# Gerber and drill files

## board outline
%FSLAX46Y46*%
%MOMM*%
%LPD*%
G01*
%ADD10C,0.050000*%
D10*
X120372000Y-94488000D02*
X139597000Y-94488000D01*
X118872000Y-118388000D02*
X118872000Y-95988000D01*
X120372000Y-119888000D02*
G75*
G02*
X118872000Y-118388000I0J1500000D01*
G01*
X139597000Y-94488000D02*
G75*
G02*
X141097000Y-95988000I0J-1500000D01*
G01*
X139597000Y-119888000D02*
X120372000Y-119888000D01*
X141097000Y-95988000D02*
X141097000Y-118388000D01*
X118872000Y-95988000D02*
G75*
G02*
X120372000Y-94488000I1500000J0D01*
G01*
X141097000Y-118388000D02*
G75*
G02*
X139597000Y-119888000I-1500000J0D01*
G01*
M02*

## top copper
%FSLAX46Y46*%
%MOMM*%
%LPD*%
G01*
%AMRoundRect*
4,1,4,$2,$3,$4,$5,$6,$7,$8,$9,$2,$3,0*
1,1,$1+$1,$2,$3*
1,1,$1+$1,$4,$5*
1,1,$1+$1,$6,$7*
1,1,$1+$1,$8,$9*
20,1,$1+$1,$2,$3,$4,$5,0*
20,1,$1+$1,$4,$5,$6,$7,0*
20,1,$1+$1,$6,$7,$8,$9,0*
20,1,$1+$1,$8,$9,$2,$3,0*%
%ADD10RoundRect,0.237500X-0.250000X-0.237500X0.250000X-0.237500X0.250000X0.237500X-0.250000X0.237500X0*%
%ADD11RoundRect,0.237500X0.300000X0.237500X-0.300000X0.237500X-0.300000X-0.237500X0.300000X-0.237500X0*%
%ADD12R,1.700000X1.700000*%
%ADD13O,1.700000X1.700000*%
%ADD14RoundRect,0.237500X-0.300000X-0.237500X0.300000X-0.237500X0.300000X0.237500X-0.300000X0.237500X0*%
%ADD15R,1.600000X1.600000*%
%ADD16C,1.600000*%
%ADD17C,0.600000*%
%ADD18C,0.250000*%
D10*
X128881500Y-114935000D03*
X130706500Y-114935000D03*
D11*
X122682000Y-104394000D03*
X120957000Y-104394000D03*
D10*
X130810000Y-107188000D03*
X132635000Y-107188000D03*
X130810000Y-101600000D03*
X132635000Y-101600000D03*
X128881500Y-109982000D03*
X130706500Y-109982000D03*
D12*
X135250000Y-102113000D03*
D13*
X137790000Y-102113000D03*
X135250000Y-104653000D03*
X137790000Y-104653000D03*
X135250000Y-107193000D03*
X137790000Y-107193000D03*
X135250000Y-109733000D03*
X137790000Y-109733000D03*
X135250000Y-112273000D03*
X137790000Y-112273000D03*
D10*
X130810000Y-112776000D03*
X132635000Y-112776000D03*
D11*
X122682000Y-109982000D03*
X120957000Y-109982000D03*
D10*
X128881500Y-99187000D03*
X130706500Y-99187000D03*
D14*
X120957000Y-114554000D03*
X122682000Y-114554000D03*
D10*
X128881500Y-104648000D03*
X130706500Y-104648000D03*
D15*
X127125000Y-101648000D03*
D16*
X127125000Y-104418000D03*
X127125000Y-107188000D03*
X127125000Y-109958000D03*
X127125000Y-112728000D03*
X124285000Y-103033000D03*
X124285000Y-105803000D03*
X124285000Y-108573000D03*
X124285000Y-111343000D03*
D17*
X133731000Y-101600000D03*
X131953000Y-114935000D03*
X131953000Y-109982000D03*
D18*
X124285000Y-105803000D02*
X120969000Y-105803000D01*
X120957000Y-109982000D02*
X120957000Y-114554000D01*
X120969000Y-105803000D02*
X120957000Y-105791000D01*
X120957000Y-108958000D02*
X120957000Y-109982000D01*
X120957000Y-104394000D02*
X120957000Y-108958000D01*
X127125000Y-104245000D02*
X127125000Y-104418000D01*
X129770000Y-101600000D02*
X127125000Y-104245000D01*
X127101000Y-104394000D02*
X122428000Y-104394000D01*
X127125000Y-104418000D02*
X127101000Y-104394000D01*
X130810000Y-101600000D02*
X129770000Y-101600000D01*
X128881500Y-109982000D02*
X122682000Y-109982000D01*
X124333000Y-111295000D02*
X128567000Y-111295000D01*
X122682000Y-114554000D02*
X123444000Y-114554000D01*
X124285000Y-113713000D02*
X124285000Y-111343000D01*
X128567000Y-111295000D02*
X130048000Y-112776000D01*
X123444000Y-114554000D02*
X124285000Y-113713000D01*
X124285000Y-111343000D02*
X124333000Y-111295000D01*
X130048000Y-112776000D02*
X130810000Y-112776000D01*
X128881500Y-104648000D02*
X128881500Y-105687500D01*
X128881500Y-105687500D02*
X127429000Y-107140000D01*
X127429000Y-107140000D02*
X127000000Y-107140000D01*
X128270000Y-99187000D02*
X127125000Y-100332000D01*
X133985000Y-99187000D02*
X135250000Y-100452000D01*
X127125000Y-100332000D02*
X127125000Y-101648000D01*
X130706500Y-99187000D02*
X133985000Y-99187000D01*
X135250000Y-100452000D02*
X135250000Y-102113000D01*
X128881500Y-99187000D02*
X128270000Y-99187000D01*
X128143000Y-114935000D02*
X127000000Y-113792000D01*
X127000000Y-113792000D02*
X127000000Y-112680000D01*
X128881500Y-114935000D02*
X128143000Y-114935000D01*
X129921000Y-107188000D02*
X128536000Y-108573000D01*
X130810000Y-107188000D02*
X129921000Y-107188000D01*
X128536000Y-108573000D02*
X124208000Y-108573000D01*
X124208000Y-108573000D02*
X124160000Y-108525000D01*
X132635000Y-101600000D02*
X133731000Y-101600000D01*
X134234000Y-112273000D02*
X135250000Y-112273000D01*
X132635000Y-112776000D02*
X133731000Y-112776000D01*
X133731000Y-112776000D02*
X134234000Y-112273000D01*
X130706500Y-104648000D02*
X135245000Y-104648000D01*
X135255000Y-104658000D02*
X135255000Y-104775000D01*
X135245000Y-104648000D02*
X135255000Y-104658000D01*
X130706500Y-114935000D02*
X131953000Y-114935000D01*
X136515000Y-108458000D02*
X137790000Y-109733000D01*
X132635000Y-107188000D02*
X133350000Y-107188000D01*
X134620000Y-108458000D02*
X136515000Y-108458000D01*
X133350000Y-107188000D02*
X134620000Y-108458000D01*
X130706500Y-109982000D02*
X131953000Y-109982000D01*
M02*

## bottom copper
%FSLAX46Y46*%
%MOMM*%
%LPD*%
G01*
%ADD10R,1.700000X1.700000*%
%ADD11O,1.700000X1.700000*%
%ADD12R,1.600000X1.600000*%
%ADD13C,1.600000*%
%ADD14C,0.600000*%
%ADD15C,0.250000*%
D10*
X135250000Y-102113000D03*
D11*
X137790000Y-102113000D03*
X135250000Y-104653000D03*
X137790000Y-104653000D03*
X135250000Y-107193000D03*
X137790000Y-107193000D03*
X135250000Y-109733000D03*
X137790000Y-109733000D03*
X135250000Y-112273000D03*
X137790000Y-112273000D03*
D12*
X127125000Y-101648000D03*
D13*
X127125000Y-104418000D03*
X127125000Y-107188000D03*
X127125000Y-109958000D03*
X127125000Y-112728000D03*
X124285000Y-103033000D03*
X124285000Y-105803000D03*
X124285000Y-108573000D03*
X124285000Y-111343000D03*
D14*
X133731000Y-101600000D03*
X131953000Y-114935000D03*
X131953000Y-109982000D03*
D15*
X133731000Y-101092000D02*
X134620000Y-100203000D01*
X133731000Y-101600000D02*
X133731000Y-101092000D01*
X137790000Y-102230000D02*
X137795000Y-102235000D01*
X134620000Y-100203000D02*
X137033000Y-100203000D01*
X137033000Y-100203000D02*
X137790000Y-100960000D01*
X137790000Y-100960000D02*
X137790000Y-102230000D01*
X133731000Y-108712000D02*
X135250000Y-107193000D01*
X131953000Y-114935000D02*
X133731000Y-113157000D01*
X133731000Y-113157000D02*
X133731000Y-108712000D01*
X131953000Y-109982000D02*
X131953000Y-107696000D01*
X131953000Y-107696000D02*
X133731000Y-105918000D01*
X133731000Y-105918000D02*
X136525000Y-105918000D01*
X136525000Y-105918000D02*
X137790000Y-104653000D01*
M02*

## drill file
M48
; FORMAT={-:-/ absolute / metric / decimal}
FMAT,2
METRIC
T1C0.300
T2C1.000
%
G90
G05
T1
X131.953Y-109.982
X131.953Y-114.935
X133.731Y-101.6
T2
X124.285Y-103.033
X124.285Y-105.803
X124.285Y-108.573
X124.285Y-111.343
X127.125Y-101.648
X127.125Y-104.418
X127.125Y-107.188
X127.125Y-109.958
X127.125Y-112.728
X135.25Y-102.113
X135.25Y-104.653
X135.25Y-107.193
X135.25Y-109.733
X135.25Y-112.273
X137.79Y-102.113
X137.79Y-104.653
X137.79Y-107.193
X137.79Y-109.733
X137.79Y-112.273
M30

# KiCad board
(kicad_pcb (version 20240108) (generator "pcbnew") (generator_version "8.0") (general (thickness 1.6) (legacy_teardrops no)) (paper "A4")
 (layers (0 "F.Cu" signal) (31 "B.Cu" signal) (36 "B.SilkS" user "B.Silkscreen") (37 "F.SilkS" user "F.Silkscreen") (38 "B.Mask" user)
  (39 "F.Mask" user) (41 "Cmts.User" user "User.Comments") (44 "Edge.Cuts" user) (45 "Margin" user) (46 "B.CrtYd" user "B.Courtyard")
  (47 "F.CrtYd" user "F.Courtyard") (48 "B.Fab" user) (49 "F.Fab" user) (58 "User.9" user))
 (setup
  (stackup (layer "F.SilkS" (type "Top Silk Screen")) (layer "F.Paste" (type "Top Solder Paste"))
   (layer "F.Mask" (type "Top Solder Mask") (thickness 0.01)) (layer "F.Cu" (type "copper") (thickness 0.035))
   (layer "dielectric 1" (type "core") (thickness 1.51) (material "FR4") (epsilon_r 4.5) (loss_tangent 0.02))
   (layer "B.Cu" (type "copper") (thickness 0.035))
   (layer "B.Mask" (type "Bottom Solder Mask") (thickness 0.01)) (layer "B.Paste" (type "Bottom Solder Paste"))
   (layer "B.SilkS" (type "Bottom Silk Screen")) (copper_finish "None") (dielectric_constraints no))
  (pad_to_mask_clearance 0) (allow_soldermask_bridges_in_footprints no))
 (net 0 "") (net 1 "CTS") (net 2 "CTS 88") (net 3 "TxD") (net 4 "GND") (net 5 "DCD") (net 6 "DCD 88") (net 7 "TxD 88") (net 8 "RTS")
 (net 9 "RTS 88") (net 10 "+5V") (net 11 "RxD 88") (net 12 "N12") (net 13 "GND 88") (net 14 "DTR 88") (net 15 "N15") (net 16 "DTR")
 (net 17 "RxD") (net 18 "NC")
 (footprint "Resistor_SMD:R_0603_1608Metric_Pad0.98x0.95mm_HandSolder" (layer "F.Cu") (at 129.794 114.935)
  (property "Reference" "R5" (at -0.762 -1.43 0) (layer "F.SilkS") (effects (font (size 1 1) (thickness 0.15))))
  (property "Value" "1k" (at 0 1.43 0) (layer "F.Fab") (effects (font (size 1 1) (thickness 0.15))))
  (pad "1" smd roundrect (at -0.9125 0) (size 0.975 0.95) (layers "F.Cu" "F.Paste" "F.Mask") (roundrect_rratio 0.25) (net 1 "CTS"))
  (pad "2" smd roundrect (at 0.9125 0) (size 0.975 0.95) (layers "F.Cu" "F.Paste" "F.Mask") (roundrect_rratio 0.25) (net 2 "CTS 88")))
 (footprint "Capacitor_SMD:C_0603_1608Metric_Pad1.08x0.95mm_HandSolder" (layer "F.Cu") (at 121.8195 104.394 180)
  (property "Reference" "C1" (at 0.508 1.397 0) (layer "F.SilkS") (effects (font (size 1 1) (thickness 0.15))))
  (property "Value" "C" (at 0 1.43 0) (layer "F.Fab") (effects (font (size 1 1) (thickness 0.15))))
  (pad "1" smd roundrect (at -0.8625 0 180) (size 1.075 0.95) (layers "F.Cu" "F.Paste" "F.Mask") (roundrect_rratio 0.25) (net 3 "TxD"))
  (pad "2" smd roundrect (at 0.8625 0 180) (size 1.075 0.95) (layers "F.Cu" "F.Paste" "F.Mask") (roundrect_rratio 0.25) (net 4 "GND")))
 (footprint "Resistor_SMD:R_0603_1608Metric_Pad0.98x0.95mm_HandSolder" (layer "F.Cu") (at 131.7225 107.188)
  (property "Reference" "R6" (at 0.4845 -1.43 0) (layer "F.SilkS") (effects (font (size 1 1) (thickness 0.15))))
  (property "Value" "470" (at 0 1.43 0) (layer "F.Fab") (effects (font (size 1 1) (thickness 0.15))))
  (pad "1" smd roundrect (at -0.9125 0) (size 0.975 0.95) (layers "F.Cu" "F.Paste" "F.Mask") (roundrect_rratio 0.25) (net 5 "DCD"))
  (pad "2" smd roundrect (at 0.9125 0) (size 0.975 0.95) (layers "F.Cu" "F.Paste" "F.Mask") (roundrect_rratio 0.25) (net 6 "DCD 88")))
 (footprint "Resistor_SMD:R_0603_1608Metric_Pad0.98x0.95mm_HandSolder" (layer "F.Cu") (at 131.7225 101.6)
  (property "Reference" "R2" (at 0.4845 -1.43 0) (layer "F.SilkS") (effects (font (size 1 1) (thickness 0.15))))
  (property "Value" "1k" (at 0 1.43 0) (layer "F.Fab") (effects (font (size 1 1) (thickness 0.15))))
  (pad "1" smd roundrect (at -0.9125 0) (size 0.975 0.95) (layers "F.Cu" "F.Paste" "F.Mask") (roundrect_rratio 0.25) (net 3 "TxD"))
  (pad "2" smd roundrect (at 0.9125 0) (size 0.975 0.95) (layers "F.Cu" "F.Paste" "F.Mask") (roundrect_rratio 0.25) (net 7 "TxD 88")))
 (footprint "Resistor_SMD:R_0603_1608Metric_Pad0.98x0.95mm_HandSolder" (layer "F.Cu") (at 129.794 109.982)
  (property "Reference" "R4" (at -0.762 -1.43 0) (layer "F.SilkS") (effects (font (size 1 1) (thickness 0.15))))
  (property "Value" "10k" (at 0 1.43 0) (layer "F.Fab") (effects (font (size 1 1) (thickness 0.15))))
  (pad "1" smd roundrect (at -0.9125 0) (size 0.975 0.95) (layers "F.Cu" "F.Paste" "F.Mask") (roundrect_rratio 0.25) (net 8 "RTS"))
  (pad "2" smd roundrect (at 0.9125 0) (size 0.975 0.95) (layers "F.Cu" "F.Paste" "F.Mask") (roundrect_rratio 0.25) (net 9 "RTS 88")))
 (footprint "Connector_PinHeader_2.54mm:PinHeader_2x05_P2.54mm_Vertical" (layer "F.Cu") (at 135.25 102.113)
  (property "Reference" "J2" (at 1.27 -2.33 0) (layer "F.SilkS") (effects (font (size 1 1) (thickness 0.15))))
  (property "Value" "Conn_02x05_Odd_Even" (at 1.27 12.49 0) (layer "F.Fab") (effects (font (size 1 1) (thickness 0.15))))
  (pad "1" thru_hole rect (at 0 0) (size 1.7 1.7) (drill 1) (layers "*.Cu" "*.Mask") (remove_unused_layers no) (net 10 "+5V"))
  (pad "2" thru_hole oval (at 2.54 0) (size 1.7 1.7) (drill 1) (layers "*.Cu" "*.Mask") (remove_unused_layers no) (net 7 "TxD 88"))
  (pad "3" thru_hole oval (at 0 2.54) (size 1.7 1.7) (drill 1) (layers "*.Cu" "*.Mask") (remove_unused_layers no) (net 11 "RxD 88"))
  (pad "4" thru_hole oval (at 2.54 2.54) (size 1.7 1.7) (drill 1) (layers "*.Cu" "*.Mask") (remove_unused_layers no) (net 9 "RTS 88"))
  (pad "5" thru_hole oval (at 0 5.08) (size 1.7 1.7) (drill 1) (layers "*.Cu" "*.Mask") (remove_unused_layers no) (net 2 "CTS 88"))
  (pad "6" thru_hole oval (at 2.54 5.08) (size 1.7 1.7) (drill 1) (layers "*.Cu" "*.Mask") (remove_unused_layers no) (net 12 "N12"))
  (pad "7" thru_hole oval (at 0 7.62) (size 1.7 1.7) (drill 1) (layers "*.Cu" "*.Mask") (remove_unused_layers no) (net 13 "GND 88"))
  (pad "8" thru_hole oval (at 2.54 7.62) (size 1.7 1.7) (drill 1) (layers "*.Cu" "*.Mask") (remove_unused_layers no) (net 6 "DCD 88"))
  (pad "9" thru_hole oval (at 0 10.16) (size 1.7 1.7) (drill 1) (layers "*.Cu" "*.Mask") (remove_unused_layers no) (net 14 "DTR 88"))
  (pad "10" thru_hole oval (at 2.54 10.16) (size 1.7 1.7) (drill 1) (layers "*.Cu" "*.Mask") (remove_unused_layers no) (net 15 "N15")))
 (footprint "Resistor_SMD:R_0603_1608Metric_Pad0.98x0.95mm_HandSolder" (layer "F.Cu") (at 131.7225 112.776)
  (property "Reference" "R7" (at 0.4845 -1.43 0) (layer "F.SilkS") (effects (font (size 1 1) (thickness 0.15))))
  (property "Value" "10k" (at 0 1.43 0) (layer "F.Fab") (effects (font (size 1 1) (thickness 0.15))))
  (pad "1" smd roundrect (at -0.9125 0) (size 0.975 0.95) (layers "F.Cu" "F.Paste" "F.Mask") (roundrect_rratio 0.25) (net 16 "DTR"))
  (pad "2" smd roundrect (at 0.9125 0) (size 0.975 0.95) (layers "F.Cu" "F.Paste" "F.Mask") (roundrect_rratio 0.25) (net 14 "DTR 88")))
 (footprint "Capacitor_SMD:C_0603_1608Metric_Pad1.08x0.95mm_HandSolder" (layer "F.Cu") (at 121.8195 109.982 180)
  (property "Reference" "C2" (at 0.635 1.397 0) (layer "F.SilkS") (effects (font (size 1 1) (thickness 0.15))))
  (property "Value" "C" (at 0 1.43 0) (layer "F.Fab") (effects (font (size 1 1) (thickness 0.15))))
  (pad "1" smd roundrect (at -0.8625 0 180) (size 1.075 0.95) (layers "F.Cu" "F.Paste" "F.Mask") (roundrect_rratio 0.25) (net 8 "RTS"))
  (pad "2" smd roundrect (at 0.8625 0 180) (size 1.075 0.95) (layers "F.Cu" "F.Paste" "F.Mask") (roundrect_rratio 0.25) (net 4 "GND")))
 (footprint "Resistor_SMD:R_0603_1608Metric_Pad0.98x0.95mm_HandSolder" (layer "F.Cu") (at 129.794 99.187)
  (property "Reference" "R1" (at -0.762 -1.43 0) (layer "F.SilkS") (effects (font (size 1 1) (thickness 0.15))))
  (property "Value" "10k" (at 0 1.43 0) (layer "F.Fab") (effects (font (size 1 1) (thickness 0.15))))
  (pad "1" smd roundrect (at -0.9125 0) (size 0.975 0.95) (layers "F.Cu" "F.Paste" "F.Mask") (roundrect_rratio 0.25) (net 10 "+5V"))
  (pad "2" smd roundrect (at 0.9125 0) (size 0.975 0.95) (layers "F.Cu" "F.Paste" "F.Mask") (roundrect_rratio 0.25) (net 10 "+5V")))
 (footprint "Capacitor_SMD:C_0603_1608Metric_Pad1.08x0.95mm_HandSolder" (layer "F.Cu") (at 121.8195 114.554)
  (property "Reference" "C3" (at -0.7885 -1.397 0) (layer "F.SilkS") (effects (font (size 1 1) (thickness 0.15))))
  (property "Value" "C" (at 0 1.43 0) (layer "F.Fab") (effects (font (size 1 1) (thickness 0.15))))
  (pad "1" smd roundrect (at -0.8625 0) (size 1.075 0.95) (layers "F.Cu" "F.Paste" "F.Mask") (roundrect_rratio 0.25) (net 4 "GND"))
  (pad "2" smd roundrect (at 0.8625 0) (size 1.075 0.95) (layers "F.Cu" "F.Paste" "F.Mask") (roundrect_rratio 0.25) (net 16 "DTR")))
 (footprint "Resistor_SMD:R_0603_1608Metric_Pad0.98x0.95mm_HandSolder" (layer "F.Cu") (at 129.794 104.648)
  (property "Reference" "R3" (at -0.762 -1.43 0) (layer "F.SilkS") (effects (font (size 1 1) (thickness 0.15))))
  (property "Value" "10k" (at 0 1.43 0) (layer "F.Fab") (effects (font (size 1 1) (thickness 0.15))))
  (pad "1" smd roundrect (at -0.9125 0) (size 0.975 0.95) (layers "F.Cu" "F.Paste" "F.Mask") (roundrect_rratio 0.25) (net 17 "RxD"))
  (pad "2" smd roundrect (at 0.9125 0) (size 0.975 0.95) (layers "F.Cu" "F.Paste" "F.Mask") (roundrect_rratio 0.25) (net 11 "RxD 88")))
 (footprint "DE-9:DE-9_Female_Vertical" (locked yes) (layer "B.Cu") (at 127.125 101.648 90)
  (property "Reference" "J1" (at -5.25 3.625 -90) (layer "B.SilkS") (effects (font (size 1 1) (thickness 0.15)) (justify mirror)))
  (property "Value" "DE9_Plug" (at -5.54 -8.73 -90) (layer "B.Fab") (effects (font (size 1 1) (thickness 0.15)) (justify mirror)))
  (pad "1" thru_hole rect (at 0 0 90) (size 1.6 1.6) (drill 1) (layers "*.Cu" "*.Mask") (remove_unused_layers no) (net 10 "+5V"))
  (pad "2" thru_hole circle (at -2.77 0 90) (size 1.6 1.6) (drill 1) (layers "*.Cu" "*.Mask") (remove_unused_layers no) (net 3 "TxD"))
  (pad "3" thru_hole circle (at -5.54 0 90) (size 1.6 1.6) (drill 1) (layers "*.Cu" "*.Mask") (remove_unused_layers no) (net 17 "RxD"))
  (pad "4" thru_hole circle (at -8.31 0 90) (size 1.6 1.6) (drill 1) (layers "*.Cu" "*.Mask") (remove_unused_layers no) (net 8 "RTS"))
  (pad "5" thru_hole circle (at -11.08 0 90) (size 1.6 1.6) (drill 1) (layers "*.Cu" "*.Mask") (remove_unused_layers no) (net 1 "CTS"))
  (pad "6" thru_hole circle (at -1.385 -2.84 90) (size 1.6 1.6) (drill 1) (layers "*.Cu" "*.Mask") (remove_unused_layers no) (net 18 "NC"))
  (pad "7" thru_hole circle (at -4.155 -2.84 90) (size 1.6 1.6) (drill 1) (layers "*.Cu" "*.Mask") (remove_unused_layers no) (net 4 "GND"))
  (pad "8" thru_hole circle (at -6.925 -2.84 90) (size 1.6 1.6) (drill 1) (layers "*.Cu" "*.Mask") (remove_unused_layers no) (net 5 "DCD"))
  (pad "9" thru_hole circle (at -9.695 -2.84 90) (size 1.6 1.6) (drill 1) (layers "*.Cu" "*.Mask") (remove_unused_layers no) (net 16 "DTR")))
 (gr_line (start 120.372 94.488) (end 139.597 94.488) (stroke (width 0.05) (type default)) (layer "Edge.Cuts"))
 (gr_line (start 118.872 118.388) (end 118.872 95.988) (stroke (width 0.05) (type default)) (layer "Edge.Cuts"))
 (gr_arc (start 120.372 119.888) (mid 119.31134 119.44866) (end 118.872 118.388) (stroke (width 0.05) (type default)) (layer "Edge.Cuts"))
 (gr_arc (start 139.597 94.488) (mid 140.65766 94.92734) (end 141.097 95.988) (stroke (width 0.05) (type default)) (layer "Edge.Cuts"))
 (gr_line (start 139.597 119.888) (end 120.372 119.888) (stroke (width 0.05) (type default)) (layer "Edge.Cuts"))
 (gr_line (start 141.097 95.988) (end 141.097 118.388) (stroke (width 0.05) (type default)) (layer "Edge.Cuts"))
 (gr_arc (start 118.872 95.988) (mid 119.31134 94.92734) (end 120.372 94.488) (stroke (width 0.05) (type default)) (layer "Edge.Cuts"))
 (gr_arc (start 141.097 118.388) (mid 140.65766 119.44866) (end 139.597 119.888) (stroke (width 0.05) (type default)) (layer "Edge.Cuts"))
 (segment (start 124.285 105.803) (end 120.969 105.803) (width 0.25) (layer "F.Cu") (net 4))
 (segment (start 120.957 109.982) (end 120.957 114.554) (width 0.25) (layer "F.Cu") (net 4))
 (segment (start 120.969 105.803) (end 120.957 105.791) (width 0.25) (layer "F.Cu") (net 4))
 (segment (start 120.957 108.958) (end 120.957 109.982) (width 0.25) (layer "F.Cu") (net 4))
 (segment (start 120.957 104.394) (end 120.957 108.958) (width 0.25) (layer "F.Cu") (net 4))
 (segment (start 127.125 104.245) (end 127.125 104.418) (width 0.25) (layer "F.Cu") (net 3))
 (segment (start 129.77 101.6) (end 127.125 104.245) (width 0.25) (layer "F.Cu") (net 3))
 (segment (start 127.101 104.394) (end 122.428 104.394) (width 0.25) (layer "F.Cu") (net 3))
 (segment (start 127.125 104.418) (end 127.101 104.394) (width 0.25) (layer "F.Cu") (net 3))
 (segment (start 130.81 101.6) (end 129.77 101.6) (width 0.25) (layer "F.Cu") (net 3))
 (segment (start 128.8815 109.982) (end 122.682 109.982) (width 0.25) (layer "F.Cu") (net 8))
 (segment (start 124.333 111.295) (end 128.567 111.295) (width 0.25) (layer "F.Cu") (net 16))
 (segment (start 122.682 114.554) (end 123.444 114.554) (width 0.25) (layer "F.Cu") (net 16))
 (segment (start 124.285 113.713) (end 124.285 111.343) (width 0.25) (layer "F.Cu") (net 16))
 (segment (start 128.567 111.295) (end 130.048 112.776) (width 0.25) (layer "F.Cu") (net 16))
 (segment (start 123.444 114.554) (end 124.285 113.713) (width 0.25) (layer "F.Cu") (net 16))
 (segment (start 124.285 111.343) (end 124.333 111.295) (width 0.25) (layer "F.Cu") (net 16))
 (segment (start 130.048 112.776) (end 130.81 112.776) (width 0.25) (layer "F.Cu") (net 16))
 (segment (start 128.8815 104.648) (end 128.8815 105.6875) (width 0.25) (layer "F.Cu") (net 17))
 (segment (start 128.8815 105.6875) (end 127.429 107.14) (width 0.25) (layer "F.Cu") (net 17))
 (segment (start 127.429 107.14) (end 127 107.14) (width 0.25) (layer "F.Cu") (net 17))
 (segment (start 128.27 99.187) (end 127.125 100.332) (width 0.25) (layer "F.Cu") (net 10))
 (segment (start 133.985 99.187) (end 135.25 100.452) (width 0.25) (layer "F.Cu") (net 10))
 (segment (start 127.125 100.332) (end 127.125 101.648) (width 0.25) (layer "F.Cu") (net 10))
 (segment (start 130.7065 99.187) (end 133.985 99.187) (width 0.25) (layer "F.Cu") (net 10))
 (segment (start 135.25 100.452) (end 135.25 102.113) (width 0.25) (layer "F.Cu") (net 10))
 (segment (start 128.8815 99.187) (end 128.27 99.187) (width 0.25) (layer "F.Cu") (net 10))
 (segment (start 128.143 114.935) (end 127 113.792) (width 0.25) (layer "F.Cu") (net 1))
 (segment (start 127 113.792) (end 127 112.68) (width 0.25) (layer "F.Cu") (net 1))
 (segment (start 128.8815 114.935) (end 128.143 114.935) (width 0.25) (layer "F.Cu") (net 1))
 (segment (start 129.921 107.188) (end 128.536 108.573) (width 0.25) (layer "F.Cu") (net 5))
 (segment (start 130.81 107.188) (end 129.921 107.188) (width 0.25) (layer "F.Cu") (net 5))
 (segment (start 128.536 108.573) (end 124.208 108.573) (width 0.25) (layer "F.Cu") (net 5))
 (segment (start 124.208 108.573) (end 124.16 108.525) (width 0.25) (layer "F.Cu") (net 5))
 (segment (start 132.635 101.6) (end 133.731 101.6) (width 0.25) (layer "F.Cu") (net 7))
 (via (at 133.731 101.6) (size 0.6) (drill 0.3) (layers "F.Cu" "B.Cu") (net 7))
 (segment (start 133.731 101.092) (end 134.62 100.203) (width 0.25) (layer "B.Cu") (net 7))
 (segment (start 133.731 101.6) (end 133.731 101.092) (width 0.25) (layer "B.Cu") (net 7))
 (segment (start 137.79 102.23) (end 137.795 102.235) (width 0.25) (layer "B.Cu") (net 7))
 (segment (start 134.62 100.203) (end 137.033 100.203) (width 0.25) (layer "B.Cu") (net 7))
 (segment (start 137.033 100.203) (end 137.79 100.96) (width 0.25) (layer "B.Cu") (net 7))
 (segment (start 137.79 100.96) (end 137.79 102.23) (width 0.25) (layer "B.Cu") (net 7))
 (segment (start 134.234 112.273) (end 135.25 112.273) (width 0.25) (layer "F.Cu") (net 14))
 (segment (start 132.635 112.776) (end 133.731 112.776) (width 0.25) (layer "F.Cu") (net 14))
 (segment (start 133.731 112.776) (end 134.234 112.273) (width 0.25) (layer "F.Cu") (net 14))
 (segment (start 130.7065 104.648) (end 135.245 104.648) (width 0.25) (layer "F.Cu") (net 11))
 (segment (start 135.255 104.658) (end 135.255 104.775) (width 0.25) (layer "F.Cu") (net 11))
 (segment (start 135.245 104.648) (end 135.255 104.658) (width 0.25) (layer "F.Cu") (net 11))
 (segment (start 130.7065 114.935) (end 131.953 114.935) (width 0.25) (layer "F.Cu") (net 2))
 (via (at 131.953 114.935) (size 0.6) (drill 0.3) (layers "F.Cu" "B.Cu") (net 2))
 (segment (start 133.731 108.712) (end 135.25 107.193) (width 0.25) (layer "B.Cu") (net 2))
 (segment (start 131.953 114.935) (end 133.731 113.157) (width 0.25) (layer "B.Cu") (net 2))
 (segment (start 133.731 113.157) (end 133.731 108.712) (width 0.25) (layer "B.Cu") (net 2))
 (segment (start 136.515 108.458) (end 137.79 109.733) (width 0.25) (layer "F.Cu") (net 6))
 (segment (start 132.635 107.188) (end 133.35 107.188) (width 0.25) (layer "F.Cu") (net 6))
 (segment (start 134.62 108.458) (end 136.515 108.458) (width 0.25) (layer "F.Cu") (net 6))
 (segment (start 133.35 107.188) (end 134.62 108.458) (width 0.25) (layer "F.Cu") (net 6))
 (segment (start 130.7065 109.982) (end 131.953 109.982) (width 0.25) (layer "F.Cu") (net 9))
 (via (at 131.953 109.982) (size 0.6) (drill 0.3) (layers "F.Cu" "B.Cu") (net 9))
 (segment (start 131.953 109.982) (end 131.953 107.696) (width 0.25) (layer "B.Cu") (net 9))
 (segment (start 131.953 107.696) (end 133.731 105.918) (width 0.25) (layer "B.Cu") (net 9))
 (segment (start 133.731 105.918) (end 136.525 105.918) (width 0.25) (layer "B.Cu") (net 9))
 (segment (start 136.525 105.918) (end 137.79 104.653) (width 0.25) (layer "B.Cu") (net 9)))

